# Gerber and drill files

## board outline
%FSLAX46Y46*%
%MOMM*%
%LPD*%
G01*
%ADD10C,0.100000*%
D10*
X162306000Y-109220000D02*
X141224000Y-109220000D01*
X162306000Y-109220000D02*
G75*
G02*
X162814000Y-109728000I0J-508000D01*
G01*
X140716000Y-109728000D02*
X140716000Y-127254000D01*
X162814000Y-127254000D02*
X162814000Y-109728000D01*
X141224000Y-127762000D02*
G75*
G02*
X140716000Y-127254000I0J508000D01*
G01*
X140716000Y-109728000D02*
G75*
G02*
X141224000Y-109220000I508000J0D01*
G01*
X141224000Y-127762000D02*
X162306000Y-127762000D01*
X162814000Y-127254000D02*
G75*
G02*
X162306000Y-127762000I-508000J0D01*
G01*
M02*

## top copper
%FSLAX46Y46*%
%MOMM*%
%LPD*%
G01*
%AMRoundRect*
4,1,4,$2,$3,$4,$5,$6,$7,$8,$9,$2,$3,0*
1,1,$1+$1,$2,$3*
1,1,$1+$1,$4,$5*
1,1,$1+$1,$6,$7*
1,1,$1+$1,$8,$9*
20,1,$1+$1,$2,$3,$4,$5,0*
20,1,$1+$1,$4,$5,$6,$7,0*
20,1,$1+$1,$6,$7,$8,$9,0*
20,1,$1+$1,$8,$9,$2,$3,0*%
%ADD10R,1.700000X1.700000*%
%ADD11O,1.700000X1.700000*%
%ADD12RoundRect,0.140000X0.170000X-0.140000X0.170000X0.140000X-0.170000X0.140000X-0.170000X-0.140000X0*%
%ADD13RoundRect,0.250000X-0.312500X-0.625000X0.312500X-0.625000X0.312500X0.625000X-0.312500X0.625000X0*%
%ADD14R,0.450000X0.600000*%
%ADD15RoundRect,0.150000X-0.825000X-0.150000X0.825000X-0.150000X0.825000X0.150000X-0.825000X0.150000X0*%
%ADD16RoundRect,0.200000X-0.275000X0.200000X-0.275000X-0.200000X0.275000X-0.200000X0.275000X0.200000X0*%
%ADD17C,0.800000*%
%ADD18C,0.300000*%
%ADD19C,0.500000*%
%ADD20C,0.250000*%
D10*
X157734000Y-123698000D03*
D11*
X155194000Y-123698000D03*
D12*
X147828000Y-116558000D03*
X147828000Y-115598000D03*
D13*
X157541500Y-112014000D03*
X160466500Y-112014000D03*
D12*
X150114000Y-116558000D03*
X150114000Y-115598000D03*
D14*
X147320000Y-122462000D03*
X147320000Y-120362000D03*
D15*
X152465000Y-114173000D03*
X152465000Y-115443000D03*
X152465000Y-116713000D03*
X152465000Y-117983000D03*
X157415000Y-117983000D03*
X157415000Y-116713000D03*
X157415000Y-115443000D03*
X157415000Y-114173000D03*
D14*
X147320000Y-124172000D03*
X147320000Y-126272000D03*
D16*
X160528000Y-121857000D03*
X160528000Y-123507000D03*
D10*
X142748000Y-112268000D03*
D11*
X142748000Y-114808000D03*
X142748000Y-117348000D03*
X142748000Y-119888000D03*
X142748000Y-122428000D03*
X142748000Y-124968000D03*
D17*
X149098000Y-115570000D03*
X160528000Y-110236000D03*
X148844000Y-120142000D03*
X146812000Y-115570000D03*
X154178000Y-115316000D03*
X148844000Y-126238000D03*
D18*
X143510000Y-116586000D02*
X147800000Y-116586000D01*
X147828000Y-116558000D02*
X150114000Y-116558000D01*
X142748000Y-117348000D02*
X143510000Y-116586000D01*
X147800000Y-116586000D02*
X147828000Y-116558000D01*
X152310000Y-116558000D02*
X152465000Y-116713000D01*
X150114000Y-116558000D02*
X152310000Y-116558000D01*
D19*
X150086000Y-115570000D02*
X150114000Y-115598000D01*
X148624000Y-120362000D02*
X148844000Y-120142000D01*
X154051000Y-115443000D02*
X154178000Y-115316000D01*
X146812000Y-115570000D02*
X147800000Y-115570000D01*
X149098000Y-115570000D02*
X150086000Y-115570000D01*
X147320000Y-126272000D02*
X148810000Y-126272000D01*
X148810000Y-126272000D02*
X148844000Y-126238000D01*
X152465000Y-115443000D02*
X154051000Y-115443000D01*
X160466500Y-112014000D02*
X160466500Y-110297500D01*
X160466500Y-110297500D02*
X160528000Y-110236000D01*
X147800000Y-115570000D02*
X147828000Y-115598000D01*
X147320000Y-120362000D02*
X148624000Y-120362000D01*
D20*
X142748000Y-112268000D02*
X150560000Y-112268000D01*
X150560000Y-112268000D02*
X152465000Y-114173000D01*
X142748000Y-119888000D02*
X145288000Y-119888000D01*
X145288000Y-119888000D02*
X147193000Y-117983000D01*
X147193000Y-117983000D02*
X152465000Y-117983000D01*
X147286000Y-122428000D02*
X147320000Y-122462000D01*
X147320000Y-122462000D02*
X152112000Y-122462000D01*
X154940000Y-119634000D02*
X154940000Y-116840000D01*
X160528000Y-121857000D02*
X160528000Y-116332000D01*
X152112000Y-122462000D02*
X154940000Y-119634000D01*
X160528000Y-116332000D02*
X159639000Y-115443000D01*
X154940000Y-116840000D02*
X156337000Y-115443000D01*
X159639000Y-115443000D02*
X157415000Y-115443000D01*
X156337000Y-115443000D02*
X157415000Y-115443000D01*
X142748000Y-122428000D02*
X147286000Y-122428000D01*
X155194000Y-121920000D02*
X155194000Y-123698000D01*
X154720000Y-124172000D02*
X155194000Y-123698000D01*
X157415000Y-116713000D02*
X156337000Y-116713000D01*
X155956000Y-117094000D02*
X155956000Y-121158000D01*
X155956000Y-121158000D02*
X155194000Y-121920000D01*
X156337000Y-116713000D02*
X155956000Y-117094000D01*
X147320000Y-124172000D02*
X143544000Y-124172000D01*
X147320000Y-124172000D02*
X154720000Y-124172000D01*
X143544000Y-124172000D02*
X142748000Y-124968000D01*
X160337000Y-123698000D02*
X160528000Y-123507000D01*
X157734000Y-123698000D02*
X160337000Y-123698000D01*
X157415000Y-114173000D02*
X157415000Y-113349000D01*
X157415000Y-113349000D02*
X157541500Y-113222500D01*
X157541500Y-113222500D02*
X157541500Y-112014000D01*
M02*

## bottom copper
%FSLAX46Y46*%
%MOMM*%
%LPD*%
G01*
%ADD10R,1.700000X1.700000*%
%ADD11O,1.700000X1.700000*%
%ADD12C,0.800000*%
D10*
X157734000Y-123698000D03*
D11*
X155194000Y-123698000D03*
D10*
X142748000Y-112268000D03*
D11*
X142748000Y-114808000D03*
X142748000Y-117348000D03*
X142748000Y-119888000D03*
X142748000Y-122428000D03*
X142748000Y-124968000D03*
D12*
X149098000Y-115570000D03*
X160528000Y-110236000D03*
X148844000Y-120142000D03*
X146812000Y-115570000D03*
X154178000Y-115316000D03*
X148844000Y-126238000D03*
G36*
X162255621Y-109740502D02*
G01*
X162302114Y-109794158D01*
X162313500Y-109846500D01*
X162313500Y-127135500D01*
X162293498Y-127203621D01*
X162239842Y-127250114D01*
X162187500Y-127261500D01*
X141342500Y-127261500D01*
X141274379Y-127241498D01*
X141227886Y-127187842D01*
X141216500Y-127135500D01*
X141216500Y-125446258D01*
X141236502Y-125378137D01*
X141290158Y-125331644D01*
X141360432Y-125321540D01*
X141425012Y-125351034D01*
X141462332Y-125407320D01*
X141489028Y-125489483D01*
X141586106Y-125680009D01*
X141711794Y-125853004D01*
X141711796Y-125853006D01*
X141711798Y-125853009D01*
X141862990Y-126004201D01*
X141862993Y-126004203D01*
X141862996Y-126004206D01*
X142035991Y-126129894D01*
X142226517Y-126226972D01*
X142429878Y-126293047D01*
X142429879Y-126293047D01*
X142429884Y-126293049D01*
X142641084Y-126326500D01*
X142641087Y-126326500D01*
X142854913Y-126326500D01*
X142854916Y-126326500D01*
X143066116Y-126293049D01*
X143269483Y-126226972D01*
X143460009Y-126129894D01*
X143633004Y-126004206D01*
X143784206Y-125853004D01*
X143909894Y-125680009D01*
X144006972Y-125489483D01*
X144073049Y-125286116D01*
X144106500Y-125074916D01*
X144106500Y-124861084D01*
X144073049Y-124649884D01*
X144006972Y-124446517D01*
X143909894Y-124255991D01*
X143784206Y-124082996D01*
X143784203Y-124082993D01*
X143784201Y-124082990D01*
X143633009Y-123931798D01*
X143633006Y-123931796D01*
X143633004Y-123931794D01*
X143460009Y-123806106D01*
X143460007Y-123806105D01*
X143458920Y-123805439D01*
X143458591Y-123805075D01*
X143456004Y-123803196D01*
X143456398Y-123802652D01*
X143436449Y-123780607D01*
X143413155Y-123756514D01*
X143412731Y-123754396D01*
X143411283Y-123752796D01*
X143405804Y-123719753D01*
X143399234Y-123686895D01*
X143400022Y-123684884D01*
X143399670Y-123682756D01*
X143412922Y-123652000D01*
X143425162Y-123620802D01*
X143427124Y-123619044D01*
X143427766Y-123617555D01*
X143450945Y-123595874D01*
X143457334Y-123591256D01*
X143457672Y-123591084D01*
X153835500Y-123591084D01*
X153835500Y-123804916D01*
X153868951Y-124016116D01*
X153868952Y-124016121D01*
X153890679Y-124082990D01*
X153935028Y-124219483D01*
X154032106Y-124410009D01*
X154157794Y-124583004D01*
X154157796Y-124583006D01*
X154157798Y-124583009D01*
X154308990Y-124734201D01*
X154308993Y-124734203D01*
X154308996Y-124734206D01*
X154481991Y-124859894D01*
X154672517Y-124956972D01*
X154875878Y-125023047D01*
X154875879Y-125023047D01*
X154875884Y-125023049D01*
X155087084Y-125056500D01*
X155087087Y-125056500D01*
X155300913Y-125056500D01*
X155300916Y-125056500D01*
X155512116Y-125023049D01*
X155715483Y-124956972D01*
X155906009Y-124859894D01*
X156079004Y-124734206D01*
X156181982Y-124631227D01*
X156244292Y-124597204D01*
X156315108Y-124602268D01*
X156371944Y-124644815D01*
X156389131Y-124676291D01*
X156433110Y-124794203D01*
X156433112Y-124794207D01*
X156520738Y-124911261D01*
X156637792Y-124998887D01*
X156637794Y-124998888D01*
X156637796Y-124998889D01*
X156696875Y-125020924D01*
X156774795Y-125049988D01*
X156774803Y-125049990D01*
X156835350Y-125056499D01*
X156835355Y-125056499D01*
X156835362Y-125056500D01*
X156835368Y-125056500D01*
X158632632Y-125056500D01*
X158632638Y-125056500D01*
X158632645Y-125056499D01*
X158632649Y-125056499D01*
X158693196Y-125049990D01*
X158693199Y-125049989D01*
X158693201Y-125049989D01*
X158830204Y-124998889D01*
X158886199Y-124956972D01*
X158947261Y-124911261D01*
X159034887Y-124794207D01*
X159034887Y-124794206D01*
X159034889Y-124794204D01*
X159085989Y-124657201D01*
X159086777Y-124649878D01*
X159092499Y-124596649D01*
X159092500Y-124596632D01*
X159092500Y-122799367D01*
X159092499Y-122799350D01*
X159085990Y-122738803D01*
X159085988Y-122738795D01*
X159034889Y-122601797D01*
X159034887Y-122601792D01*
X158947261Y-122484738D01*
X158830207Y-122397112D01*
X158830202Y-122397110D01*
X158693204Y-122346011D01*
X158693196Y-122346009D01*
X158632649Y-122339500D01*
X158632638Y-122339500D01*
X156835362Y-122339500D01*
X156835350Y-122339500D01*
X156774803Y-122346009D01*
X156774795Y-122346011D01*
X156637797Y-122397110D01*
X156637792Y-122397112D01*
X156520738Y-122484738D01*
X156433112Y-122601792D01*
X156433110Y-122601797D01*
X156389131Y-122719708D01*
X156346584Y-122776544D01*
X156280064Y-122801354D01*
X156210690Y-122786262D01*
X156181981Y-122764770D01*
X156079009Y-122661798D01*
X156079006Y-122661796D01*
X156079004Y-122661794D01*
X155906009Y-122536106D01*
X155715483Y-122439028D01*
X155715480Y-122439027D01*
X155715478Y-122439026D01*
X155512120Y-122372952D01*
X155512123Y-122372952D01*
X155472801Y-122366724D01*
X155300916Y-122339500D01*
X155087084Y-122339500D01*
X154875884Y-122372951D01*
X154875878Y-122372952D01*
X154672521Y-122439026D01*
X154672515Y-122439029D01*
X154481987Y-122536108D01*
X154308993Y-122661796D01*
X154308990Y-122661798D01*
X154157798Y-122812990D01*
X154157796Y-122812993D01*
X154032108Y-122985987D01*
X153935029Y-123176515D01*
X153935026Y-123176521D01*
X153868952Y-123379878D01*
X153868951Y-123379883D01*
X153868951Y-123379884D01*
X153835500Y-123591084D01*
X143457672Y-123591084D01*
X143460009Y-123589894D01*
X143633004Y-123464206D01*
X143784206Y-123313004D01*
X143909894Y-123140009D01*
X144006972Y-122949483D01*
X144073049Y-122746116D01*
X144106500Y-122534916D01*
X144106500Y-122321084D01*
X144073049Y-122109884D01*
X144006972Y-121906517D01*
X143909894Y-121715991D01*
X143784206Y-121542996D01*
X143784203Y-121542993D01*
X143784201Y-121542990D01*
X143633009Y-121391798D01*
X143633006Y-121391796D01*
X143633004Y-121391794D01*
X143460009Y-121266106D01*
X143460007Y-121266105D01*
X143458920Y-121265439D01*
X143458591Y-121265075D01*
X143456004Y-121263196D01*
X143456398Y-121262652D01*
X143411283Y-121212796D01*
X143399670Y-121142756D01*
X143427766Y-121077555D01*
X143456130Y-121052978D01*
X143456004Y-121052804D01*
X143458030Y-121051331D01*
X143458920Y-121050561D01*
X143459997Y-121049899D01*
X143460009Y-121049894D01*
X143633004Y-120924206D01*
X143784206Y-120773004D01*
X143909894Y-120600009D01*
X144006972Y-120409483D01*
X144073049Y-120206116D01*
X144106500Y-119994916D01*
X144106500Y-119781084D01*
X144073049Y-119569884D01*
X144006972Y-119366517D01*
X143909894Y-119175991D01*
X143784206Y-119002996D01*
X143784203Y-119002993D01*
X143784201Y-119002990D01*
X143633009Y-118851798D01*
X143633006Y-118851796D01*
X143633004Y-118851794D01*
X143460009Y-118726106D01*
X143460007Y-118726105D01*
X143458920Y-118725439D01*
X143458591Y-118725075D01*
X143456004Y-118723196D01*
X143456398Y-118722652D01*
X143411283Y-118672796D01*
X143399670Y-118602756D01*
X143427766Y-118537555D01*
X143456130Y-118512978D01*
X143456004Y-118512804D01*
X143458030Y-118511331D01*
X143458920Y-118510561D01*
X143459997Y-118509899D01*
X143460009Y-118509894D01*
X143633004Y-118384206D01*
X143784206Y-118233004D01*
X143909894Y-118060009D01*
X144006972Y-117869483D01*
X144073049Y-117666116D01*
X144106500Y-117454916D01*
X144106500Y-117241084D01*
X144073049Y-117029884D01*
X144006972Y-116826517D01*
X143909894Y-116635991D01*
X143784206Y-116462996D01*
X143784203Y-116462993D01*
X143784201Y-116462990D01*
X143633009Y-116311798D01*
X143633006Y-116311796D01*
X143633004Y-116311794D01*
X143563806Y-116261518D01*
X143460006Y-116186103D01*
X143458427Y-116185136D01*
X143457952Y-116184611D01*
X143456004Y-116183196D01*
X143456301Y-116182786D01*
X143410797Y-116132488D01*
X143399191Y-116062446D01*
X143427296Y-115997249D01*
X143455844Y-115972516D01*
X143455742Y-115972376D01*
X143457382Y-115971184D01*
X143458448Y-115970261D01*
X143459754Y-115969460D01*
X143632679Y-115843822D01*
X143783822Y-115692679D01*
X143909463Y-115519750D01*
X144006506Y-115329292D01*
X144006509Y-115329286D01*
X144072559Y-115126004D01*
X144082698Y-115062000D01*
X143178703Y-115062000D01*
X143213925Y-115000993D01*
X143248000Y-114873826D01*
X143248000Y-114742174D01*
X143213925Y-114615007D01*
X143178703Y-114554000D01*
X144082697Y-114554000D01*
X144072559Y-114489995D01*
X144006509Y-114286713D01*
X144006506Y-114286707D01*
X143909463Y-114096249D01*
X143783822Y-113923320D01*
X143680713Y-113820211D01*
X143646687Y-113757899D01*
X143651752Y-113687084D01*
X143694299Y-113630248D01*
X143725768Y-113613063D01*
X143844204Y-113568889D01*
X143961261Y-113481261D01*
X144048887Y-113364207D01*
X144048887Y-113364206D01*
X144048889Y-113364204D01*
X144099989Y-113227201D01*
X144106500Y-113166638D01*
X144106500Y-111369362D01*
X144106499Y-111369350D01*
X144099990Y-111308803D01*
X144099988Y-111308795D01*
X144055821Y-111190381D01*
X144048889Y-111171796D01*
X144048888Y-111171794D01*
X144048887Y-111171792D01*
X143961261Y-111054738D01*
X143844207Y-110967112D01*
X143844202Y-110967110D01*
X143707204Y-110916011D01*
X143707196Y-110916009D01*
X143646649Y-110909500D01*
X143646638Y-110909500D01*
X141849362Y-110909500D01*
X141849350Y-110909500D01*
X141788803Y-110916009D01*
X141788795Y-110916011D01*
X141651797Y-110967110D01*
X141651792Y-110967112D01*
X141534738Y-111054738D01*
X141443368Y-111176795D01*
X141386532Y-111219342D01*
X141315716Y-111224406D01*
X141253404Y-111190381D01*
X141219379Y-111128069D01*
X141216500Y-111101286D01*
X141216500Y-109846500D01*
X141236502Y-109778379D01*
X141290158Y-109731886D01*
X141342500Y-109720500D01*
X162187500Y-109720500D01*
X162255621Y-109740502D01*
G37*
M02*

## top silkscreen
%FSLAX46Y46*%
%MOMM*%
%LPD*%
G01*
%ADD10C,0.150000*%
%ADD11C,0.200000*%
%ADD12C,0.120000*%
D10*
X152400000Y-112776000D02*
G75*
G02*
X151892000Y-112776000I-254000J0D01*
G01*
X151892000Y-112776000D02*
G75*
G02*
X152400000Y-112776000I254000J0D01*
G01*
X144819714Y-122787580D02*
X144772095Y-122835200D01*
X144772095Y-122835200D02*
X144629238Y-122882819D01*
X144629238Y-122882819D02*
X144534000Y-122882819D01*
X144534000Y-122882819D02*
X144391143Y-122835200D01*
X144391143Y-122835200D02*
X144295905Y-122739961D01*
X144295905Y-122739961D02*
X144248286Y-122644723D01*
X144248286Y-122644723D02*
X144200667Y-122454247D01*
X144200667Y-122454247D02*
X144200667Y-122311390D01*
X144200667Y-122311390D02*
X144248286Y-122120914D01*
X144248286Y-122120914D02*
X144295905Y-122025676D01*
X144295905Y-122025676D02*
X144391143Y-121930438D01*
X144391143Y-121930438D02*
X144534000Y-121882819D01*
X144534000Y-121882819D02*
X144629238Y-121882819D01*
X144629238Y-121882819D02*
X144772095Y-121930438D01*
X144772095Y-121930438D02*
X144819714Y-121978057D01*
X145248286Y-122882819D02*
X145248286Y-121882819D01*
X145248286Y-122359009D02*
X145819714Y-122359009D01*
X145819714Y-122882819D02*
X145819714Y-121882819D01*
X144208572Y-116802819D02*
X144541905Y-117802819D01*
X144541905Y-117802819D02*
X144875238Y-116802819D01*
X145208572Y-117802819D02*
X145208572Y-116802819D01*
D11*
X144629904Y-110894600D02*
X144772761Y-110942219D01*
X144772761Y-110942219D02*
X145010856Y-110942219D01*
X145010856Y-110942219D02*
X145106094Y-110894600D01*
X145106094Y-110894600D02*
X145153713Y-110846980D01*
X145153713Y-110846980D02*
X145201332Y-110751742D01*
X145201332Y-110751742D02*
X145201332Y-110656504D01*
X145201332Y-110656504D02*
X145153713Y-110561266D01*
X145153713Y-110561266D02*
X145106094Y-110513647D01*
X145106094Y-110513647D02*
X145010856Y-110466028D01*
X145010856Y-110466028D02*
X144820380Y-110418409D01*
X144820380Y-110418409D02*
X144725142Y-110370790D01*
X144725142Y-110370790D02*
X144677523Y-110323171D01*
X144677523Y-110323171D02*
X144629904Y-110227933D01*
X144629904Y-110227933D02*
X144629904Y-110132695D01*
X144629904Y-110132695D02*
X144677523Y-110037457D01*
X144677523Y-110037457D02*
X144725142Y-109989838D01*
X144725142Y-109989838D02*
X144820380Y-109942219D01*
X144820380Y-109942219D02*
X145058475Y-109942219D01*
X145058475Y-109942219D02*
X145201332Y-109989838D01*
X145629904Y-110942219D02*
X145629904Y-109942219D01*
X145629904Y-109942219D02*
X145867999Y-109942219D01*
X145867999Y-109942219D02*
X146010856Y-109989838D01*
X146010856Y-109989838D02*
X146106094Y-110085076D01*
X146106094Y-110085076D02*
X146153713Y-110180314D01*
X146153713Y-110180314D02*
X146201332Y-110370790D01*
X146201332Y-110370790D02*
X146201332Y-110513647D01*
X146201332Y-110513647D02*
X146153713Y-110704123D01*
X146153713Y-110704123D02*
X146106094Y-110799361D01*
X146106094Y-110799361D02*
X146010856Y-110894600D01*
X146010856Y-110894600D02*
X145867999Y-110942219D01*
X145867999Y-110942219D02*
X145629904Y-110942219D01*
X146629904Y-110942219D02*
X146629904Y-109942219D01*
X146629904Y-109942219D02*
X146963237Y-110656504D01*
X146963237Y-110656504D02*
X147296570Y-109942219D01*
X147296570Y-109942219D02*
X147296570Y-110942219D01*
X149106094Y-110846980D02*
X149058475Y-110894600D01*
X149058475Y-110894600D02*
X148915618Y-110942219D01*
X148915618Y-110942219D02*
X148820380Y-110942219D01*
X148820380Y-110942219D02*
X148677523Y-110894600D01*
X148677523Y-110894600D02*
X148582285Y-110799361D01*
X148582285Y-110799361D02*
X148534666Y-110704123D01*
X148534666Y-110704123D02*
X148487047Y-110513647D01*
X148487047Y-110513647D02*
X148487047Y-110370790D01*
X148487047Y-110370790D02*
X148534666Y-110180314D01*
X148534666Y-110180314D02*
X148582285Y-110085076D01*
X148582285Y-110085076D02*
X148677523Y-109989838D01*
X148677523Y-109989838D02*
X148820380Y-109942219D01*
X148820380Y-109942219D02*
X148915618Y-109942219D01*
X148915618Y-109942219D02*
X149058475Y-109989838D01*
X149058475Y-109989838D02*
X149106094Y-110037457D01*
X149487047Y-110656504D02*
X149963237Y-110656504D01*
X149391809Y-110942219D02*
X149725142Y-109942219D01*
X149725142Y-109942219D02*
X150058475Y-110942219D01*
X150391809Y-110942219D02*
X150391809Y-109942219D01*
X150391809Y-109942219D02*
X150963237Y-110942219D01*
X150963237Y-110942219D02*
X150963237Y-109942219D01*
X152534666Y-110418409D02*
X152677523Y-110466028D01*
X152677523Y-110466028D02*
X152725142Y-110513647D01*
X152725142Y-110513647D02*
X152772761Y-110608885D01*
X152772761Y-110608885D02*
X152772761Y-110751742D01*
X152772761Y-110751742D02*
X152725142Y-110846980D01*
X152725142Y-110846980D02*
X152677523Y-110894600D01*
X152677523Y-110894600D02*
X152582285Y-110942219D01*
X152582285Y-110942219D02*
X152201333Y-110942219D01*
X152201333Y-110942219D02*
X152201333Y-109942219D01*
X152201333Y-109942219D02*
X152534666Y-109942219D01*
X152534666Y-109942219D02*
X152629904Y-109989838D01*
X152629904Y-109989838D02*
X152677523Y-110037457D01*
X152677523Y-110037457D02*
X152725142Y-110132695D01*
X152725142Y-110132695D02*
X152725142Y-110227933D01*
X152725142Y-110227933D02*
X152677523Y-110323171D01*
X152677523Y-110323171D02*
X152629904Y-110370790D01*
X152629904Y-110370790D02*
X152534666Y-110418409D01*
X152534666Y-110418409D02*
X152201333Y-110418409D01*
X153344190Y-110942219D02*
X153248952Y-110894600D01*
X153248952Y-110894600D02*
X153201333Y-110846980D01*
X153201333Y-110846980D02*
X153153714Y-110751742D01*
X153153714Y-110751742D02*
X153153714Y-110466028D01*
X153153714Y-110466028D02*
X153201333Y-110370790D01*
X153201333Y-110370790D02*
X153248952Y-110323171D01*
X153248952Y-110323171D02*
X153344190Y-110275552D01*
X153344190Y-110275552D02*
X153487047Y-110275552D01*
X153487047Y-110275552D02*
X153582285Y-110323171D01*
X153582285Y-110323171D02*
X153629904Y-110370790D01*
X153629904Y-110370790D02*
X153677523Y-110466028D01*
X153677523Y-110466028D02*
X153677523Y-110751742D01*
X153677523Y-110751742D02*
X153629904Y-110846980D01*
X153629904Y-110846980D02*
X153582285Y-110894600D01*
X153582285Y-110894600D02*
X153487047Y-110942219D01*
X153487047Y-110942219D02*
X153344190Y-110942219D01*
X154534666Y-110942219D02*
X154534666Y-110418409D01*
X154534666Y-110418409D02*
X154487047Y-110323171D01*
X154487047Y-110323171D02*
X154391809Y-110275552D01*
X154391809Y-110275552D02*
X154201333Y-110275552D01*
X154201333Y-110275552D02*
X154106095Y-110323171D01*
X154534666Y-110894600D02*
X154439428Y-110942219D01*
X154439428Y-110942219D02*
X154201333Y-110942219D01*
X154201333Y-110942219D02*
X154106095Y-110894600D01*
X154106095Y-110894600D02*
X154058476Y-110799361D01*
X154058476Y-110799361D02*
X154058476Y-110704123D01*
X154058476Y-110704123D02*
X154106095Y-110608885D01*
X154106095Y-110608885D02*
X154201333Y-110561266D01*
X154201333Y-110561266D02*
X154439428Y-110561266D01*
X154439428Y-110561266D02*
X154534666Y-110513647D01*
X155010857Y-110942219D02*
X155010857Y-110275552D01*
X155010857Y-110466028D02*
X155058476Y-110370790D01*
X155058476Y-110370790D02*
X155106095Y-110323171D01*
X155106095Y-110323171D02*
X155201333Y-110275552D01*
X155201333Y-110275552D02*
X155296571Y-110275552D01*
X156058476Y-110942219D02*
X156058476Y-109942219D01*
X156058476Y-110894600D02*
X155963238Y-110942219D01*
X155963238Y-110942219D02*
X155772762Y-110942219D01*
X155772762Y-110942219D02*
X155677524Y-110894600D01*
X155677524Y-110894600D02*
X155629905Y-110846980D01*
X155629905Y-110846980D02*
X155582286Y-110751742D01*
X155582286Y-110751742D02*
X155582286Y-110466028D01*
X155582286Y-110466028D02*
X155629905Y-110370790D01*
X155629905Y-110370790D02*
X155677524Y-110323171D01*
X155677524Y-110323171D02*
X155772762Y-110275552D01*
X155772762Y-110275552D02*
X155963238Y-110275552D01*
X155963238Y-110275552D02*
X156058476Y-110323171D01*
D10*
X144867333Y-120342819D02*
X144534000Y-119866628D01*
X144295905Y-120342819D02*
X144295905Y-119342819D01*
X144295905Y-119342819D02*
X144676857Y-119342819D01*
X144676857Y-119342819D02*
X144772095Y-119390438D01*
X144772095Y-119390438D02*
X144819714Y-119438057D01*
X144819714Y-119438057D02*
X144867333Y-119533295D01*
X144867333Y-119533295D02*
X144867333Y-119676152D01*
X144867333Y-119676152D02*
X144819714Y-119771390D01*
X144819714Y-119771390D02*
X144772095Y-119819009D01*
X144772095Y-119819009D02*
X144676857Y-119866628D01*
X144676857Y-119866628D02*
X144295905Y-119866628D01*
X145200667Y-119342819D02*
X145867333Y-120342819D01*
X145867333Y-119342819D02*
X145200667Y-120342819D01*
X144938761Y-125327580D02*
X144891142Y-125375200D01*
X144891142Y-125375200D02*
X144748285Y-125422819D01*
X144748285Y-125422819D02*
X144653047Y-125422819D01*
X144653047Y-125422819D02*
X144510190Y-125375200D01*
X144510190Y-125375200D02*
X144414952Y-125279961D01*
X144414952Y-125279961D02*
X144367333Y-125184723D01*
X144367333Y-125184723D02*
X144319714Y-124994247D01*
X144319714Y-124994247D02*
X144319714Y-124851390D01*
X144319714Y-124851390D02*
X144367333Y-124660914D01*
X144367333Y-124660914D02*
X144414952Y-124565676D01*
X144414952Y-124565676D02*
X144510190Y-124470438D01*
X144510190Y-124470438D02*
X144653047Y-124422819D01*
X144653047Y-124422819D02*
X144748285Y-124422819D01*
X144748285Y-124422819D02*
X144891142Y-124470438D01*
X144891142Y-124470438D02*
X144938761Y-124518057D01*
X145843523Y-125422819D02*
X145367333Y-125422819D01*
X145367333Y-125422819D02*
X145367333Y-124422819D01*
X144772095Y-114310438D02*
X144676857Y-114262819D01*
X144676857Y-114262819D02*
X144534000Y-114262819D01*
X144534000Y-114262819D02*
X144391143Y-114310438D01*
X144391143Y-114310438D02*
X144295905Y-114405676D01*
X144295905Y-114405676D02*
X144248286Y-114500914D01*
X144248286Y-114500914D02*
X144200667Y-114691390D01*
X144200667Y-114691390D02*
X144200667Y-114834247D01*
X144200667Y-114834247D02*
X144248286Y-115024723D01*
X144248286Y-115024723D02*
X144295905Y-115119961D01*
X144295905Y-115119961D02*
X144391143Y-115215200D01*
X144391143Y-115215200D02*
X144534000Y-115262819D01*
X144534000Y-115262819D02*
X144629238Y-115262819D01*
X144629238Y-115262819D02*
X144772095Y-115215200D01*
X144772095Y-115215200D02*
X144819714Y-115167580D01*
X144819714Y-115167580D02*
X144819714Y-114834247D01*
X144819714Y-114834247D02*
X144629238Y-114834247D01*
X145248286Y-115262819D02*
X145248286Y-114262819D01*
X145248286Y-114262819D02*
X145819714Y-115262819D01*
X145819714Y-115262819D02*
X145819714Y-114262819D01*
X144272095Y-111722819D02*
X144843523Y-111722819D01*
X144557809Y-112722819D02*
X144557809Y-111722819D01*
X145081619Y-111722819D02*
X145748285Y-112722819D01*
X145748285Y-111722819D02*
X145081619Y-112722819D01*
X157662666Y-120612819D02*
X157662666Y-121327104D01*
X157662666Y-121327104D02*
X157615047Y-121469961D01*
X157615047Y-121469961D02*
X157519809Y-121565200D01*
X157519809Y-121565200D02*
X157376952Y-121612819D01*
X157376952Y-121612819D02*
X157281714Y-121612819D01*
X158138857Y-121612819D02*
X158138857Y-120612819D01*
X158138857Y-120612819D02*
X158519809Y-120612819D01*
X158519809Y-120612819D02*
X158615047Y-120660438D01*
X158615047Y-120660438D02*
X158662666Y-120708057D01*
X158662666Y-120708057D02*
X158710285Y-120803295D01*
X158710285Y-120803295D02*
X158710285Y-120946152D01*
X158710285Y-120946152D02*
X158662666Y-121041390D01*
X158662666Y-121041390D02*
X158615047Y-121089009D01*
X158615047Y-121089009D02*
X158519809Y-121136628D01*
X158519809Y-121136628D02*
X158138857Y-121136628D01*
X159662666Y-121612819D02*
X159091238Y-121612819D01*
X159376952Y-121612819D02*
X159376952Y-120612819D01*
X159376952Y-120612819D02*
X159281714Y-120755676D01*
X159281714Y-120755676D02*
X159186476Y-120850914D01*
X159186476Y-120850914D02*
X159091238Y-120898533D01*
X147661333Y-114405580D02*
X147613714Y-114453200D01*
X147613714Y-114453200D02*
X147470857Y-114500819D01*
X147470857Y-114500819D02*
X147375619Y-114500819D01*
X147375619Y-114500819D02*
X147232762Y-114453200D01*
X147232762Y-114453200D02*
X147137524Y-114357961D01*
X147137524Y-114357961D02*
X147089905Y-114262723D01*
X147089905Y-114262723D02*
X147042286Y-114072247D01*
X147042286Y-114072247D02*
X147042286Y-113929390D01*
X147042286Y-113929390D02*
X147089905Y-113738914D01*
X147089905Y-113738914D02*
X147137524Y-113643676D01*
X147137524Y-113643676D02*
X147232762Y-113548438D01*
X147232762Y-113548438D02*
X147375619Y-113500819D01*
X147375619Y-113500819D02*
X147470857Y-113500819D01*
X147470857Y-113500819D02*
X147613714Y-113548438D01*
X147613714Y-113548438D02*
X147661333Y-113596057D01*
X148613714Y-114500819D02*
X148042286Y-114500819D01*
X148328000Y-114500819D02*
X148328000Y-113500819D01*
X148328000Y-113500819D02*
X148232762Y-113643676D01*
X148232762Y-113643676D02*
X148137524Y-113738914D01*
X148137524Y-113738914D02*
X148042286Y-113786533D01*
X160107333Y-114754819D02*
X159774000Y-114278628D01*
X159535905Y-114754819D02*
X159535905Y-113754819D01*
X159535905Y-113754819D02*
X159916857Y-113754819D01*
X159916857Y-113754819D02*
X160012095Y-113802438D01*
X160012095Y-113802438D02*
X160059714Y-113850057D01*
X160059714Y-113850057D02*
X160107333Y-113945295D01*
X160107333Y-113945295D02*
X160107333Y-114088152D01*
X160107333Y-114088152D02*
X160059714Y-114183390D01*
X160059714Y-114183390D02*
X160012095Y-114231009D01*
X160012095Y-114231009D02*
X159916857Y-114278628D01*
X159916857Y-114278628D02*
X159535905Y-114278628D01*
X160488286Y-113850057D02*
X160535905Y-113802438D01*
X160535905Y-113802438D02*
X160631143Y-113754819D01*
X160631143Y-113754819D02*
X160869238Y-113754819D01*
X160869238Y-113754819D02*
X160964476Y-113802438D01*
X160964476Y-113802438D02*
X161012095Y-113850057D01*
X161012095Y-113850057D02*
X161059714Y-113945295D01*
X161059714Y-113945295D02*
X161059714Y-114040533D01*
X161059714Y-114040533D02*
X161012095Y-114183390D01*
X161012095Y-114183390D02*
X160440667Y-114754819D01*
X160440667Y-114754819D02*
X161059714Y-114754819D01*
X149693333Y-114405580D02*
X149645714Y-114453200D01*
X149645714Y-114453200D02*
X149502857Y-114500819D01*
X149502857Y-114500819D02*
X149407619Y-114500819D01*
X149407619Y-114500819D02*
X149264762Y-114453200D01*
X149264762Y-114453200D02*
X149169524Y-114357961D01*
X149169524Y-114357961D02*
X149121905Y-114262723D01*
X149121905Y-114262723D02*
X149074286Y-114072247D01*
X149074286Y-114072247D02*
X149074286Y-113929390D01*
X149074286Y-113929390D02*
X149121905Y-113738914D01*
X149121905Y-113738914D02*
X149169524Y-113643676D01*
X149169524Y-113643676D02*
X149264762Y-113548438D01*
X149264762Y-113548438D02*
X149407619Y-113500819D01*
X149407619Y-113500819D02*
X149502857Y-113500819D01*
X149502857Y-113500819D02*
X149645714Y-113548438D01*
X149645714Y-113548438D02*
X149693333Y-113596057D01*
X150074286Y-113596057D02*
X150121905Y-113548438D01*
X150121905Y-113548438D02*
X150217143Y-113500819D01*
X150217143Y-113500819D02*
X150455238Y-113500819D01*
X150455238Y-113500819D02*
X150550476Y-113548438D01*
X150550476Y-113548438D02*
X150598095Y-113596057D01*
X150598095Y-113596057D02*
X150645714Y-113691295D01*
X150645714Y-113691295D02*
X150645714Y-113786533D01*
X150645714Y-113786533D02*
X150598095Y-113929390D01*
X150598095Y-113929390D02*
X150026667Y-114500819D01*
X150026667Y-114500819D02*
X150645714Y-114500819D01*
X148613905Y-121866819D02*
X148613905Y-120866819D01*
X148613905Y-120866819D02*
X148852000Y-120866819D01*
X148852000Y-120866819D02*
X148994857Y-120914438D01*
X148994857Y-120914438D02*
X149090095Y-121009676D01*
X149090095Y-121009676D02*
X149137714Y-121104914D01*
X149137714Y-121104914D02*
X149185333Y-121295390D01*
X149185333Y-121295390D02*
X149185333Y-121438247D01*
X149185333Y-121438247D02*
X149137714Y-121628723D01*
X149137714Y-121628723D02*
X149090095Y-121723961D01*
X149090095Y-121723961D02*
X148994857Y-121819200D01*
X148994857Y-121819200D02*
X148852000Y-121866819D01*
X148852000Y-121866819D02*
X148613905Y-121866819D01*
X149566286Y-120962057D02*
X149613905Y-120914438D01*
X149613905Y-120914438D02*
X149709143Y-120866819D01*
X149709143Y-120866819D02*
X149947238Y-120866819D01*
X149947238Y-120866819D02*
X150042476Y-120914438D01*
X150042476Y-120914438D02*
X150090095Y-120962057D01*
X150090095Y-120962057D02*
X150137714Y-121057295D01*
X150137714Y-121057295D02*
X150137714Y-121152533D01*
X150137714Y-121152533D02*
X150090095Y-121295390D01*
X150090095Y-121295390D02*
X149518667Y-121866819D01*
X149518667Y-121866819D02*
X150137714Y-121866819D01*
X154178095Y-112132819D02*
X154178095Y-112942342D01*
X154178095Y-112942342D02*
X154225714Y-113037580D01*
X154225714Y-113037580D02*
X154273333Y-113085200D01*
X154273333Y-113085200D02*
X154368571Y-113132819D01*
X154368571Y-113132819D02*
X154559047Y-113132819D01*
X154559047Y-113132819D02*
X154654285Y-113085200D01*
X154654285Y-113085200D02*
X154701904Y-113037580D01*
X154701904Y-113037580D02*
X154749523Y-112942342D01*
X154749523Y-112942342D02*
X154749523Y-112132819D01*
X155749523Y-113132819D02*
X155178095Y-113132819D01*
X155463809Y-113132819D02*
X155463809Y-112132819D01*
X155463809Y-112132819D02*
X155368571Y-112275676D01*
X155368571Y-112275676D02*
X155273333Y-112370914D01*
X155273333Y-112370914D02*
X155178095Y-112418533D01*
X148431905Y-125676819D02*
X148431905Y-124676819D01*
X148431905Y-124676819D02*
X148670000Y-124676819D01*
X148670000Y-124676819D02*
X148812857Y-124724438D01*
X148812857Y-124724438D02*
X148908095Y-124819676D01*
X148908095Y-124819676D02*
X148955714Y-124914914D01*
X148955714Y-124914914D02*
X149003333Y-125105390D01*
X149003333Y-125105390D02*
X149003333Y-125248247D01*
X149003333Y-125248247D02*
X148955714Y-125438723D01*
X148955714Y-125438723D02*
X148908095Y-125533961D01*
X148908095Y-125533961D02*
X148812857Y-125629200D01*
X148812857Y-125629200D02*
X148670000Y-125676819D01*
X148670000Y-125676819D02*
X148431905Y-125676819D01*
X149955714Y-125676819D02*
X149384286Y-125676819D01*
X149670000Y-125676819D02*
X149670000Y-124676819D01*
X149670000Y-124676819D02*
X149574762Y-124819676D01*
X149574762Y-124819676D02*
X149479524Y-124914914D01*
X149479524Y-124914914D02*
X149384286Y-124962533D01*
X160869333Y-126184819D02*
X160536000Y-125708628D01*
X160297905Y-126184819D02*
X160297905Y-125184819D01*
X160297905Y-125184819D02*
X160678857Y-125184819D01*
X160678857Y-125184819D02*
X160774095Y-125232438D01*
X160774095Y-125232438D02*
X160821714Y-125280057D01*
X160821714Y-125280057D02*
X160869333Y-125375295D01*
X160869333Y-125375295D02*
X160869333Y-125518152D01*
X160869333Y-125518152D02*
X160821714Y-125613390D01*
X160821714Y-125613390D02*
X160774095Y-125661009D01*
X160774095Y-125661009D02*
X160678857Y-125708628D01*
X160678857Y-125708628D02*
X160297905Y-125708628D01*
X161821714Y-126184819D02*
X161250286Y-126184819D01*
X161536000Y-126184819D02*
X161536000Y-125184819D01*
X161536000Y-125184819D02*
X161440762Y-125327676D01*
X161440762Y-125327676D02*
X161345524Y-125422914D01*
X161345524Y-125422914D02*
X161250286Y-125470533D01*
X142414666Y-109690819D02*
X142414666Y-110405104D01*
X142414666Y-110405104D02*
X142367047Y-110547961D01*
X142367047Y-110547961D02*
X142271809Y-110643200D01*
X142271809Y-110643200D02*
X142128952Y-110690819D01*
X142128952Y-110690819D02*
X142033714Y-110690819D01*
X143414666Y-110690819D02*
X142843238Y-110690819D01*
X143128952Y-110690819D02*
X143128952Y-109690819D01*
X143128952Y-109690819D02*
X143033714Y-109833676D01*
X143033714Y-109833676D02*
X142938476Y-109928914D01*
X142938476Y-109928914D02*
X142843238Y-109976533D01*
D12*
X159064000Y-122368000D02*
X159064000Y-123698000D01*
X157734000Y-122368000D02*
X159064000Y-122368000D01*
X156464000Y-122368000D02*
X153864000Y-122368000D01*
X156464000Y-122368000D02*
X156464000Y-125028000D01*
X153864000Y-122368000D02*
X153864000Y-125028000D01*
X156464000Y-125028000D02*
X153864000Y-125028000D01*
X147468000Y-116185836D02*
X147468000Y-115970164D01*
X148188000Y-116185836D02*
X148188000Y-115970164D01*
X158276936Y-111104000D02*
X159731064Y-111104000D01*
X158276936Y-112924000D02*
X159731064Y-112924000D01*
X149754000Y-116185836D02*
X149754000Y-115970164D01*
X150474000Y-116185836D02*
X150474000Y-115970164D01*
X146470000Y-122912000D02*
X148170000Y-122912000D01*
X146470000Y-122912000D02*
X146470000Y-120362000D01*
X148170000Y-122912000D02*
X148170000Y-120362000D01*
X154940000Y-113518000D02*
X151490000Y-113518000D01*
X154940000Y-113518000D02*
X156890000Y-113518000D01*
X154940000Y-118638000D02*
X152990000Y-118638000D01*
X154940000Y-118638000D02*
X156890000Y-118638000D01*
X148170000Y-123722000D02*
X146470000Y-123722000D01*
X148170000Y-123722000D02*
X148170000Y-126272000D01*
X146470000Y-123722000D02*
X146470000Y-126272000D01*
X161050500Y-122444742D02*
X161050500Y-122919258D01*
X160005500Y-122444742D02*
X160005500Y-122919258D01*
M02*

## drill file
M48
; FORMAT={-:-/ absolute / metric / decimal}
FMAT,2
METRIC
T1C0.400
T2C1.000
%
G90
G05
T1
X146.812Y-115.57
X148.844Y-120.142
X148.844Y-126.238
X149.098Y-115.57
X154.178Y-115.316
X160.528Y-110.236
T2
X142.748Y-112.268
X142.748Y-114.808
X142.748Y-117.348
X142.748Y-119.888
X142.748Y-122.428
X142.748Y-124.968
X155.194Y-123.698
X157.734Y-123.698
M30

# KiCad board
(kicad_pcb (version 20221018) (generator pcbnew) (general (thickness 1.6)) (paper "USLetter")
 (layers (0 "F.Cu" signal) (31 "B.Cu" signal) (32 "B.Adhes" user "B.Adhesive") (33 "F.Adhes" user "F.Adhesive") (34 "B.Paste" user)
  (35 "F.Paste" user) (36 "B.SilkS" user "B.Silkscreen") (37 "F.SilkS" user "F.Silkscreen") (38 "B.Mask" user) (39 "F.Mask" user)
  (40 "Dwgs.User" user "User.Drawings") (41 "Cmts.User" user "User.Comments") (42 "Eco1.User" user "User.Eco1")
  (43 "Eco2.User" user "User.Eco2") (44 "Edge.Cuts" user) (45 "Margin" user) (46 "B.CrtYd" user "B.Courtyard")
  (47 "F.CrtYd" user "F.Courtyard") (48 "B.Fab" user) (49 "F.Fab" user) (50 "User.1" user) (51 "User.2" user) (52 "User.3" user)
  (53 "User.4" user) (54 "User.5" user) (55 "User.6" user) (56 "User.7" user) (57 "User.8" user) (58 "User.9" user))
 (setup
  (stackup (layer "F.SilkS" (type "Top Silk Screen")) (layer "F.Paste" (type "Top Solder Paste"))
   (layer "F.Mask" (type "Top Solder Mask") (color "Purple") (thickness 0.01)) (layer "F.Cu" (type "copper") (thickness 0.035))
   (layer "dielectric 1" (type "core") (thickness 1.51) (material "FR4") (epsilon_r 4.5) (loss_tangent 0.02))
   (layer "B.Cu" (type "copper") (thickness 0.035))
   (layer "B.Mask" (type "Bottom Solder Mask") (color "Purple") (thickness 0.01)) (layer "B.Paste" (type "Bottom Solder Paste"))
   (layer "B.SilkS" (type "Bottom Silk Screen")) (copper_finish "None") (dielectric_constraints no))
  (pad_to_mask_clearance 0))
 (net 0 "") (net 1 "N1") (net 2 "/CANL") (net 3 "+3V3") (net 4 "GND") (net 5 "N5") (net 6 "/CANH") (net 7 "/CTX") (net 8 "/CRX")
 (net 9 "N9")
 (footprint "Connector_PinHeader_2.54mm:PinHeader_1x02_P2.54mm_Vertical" (layer "F.Cu") (at 157.734 123.698 -90)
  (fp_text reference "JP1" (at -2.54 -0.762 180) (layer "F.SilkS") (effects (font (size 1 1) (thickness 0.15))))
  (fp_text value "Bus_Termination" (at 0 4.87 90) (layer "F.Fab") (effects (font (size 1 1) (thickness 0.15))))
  (fp_line (start -1.33 -1.33) (end 0 -1.33) (stroke (width 0.12) (type solid)) (layer "F.SilkS"))
  (fp_line (start -1.33 0) (end -1.33 -1.33) (stroke (width 0.12) (type solid)) (layer "F.SilkS"))
  (fp_line (start -1.33 1.27) (end -1.33 3.87) (stroke (width 0.12) (type solid)) (layer "F.SilkS"))
  (fp_line (start -1.33 1.27) (end 1.33 1.27) (stroke (width 0.12) (type solid)) (layer "F.SilkS"))
  (fp_line (start -1.33 3.87) (end 1.33 3.87) (stroke (width 0.12) (type solid)) (layer "F.SilkS"))
  (fp_line (start 1.33 1.27) (end 1.33 3.87) (stroke (width 0.12) (type solid)) (layer "F.SilkS"))
  (pad "1" thru_hole rect (at 0 0 270) (size 1.7 1.7) (drill 1) (layers "*.Cu" "*.Mask") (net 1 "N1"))
  (pad "2" thru_hole oval (at 0 2.54 270) (size 1.7 1.7) (drill 1) (layers "*.Cu" "*.Mask") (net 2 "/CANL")))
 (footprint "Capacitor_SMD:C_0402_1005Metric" (layer "F.Cu") (at 147.828 116.078 90)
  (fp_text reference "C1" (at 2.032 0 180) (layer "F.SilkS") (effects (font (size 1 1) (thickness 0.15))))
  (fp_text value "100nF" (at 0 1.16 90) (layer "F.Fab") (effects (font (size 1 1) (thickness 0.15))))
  (fp_line (start -0.107836 -0.36) (end 0.107836 -0.36) (stroke (width 0.12) (type solid)) (layer "F.SilkS"))
  (fp_line (start -0.107836 0.36) (end 0.107836 0.36) (stroke (width 0.12) (type solid)) (layer "F.SilkS"))
  (pad "1" smd roundrect (at -0.48 0 90) (size 0.56 0.62) (layers "F.Cu" "F.Paste" "F.Mask") (roundrect_rratio 0.25) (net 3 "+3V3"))
  (pad "2" smd roundrect (at 0.48 0 90) (size 0.56 0.62) (layers "F.Cu" "F.Paste" "F.Mask") (roundrect_rratio 0.25) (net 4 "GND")))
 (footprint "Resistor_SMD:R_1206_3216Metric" (layer "F.Cu") (at 159.004 112.014)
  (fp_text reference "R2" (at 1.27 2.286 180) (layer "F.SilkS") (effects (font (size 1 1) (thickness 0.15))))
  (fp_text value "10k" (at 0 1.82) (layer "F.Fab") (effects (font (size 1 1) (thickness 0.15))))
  (fp_line (start -0.727064 -0.91) (end 0.727064 -0.91) (stroke (width 0.12) (type solid)) (layer "F.SilkS"))
  (fp_line (start -0.727064 0.91) (end 0.727064 0.91) (stroke (width 0.12) (type solid)) (layer "F.SilkS"))
  (pad "1" smd roundrect (at -1.4625 0) (size 1.125 1.75) (layers "F.Cu" "F.Paste" "F.Mask") (roundrect_rratio 0.2222222222) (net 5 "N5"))
  (pad "2" smd roundrect (at 1.4625 0) (size 1.125 1.75) (layers "F.Cu" "F.Paste" "F.Mask") (roundrect_rratio 0.2222222222) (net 4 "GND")))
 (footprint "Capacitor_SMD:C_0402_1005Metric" (layer "F.Cu") (at 150.114 116.078 90)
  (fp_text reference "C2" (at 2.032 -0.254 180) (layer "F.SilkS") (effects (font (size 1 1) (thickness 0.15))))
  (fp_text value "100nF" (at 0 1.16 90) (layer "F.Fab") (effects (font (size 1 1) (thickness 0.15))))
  (fp_line (start -0.107836 -0.36) (end 0.107836 -0.36) (stroke (width 0.12) (type solid)) (layer "F.SilkS"))
  (fp_line (start -0.107836 0.36) (end 0.107836 0.36) (stroke (width 0.12) (type solid)) (layer "F.SilkS"))
  (pad "1" smd roundrect (at -0.48 0 90) (size 0.56 0.62) (layers "F.Cu" "F.Paste" "F.Mask") (roundrect_rratio 0.25) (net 3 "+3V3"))
  (pad "2" smd roundrect (at 0.48 0 90) (size 0.56 0.62) (layers "F.Cu" "F.Paste" "F.Mask") (roundrect_rratio 0.25) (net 4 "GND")))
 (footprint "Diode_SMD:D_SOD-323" (layer "F.Cu") (at 147.32 121.412 90)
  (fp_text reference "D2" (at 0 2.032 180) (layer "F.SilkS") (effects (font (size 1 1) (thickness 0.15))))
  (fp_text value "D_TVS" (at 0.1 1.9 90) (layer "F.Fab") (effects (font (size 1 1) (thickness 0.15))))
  (fp_line (start -1.5 -0.85) (end -1.5 0.85) (stroke (width 0.12) (type solid)) (layer "F.SilkS"))
  (fp_line (start -1.5 -0.85) (end 1.05 -0.85) (stroke (width 0.12) (type solid)) (layer "F.SilkS"))
  (fp_line (start -1.5 0.85) (end 1.05 0.85) (stroke (width 0.12) (type solid)) (layer "F.SilkS"))
  (pad "1" smd rect (at -1.05 0 90) (size 0.6 0.45) (layers "F.Cu" "F.Paste" "F.Mask") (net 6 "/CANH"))
  (pad "2" smd rect (at 1.05 0 90) (size 0.6 0.45) (layers "F.Cu" "F.Paste" "F.Mask") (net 4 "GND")))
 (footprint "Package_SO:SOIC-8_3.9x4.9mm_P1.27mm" (layer "F.Cu") (at 154.94 116.078)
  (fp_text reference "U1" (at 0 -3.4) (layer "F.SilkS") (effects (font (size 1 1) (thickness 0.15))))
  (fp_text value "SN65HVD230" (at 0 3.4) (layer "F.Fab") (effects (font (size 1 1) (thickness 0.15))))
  (fp_line (start 0 -2.56) (end -3.45 -2.56) (stroke (width 0.12) (type solid)) (layer "F.SilkS"))
  (fp_line (start 0 -2.56) (end 1.95 -2.56) (stroke (width 0.12) (type solid)) (layer "F.SilkS"))
  (fp_line (start 0 2.56) (end -1.95 2.56) (stroke (width 0.12) (type solid)) (layer "F.SilkS"))
  (fp_line (start 0 2.56) (end 1.95 2.56) (stroke (width 0.12) (type solid)) (layer "F.SilkS"))
  (pad "1" smd roundrect (at -2.475 -1.905) (size 1.95 0.6) (layers "F.Cu" "F.Paste" "F.Mask") (roundrect_rratio 0.25) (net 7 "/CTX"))
  (pad "2" smd roundrect (at -2.475 -0.635) (size 1.95 0.6) (layers "F.Cu" "F.Paste" "F.Mask") (roundrect_rratio 0.25) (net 4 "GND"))
  (pad "3" smd roundrect (at -2.475 0.635) (size 1.95 0.6) (layers "F.Cu" "F.Paste" "F.Mask") (roundrect_rratio 0.25) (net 3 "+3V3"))
  (pad "4" smd roundrect (at -2.475 1.905) (size 1.95 0.6) (layers "F.Cu" "F.Paste" "F.Mask") (roundrect_rratio 0.25) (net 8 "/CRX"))
  (pad "5" smd roundrect (at 2.475 1.905) (size 1.95 0.6) (layers "F.Cu" "F.Paste" "F.Mask") (roundrect_rratio 0.25) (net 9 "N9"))
  (pad "6" smd roundrect (at 2.475 0.635) (size 1.95 0.6) (layers "F.Cu" "F.Paste" "F.Mask") (roundrect_rratio 0.25) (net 2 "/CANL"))
  (pad "7" smd roundrect (at 2.475 -0.635) (size 1.95 0.6) (layers "F.Cu" "F.Paste" "F.Mask") (roundrect_rratio 0.25) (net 6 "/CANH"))
  (pad "8" smd roundrect (at 2.475 -1.905) (size 1.95 0.6) (layers "F.Cu" "F.Paste" "F.Mask") (roundrect_rratio 0.25) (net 5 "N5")))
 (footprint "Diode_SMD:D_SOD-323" (layer "F.Cu") (at 147.32 125.222 -90)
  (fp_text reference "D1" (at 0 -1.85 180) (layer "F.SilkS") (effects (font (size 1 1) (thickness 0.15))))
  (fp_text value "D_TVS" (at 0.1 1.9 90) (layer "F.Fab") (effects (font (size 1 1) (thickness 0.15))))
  (fp_line (start -1.5 -0.85) (end -1.5 0.85) (stroke (width 0.12) (type solid)) (layer "F.SilkS"))
  (fp_line (start -1.5 -0.85) (end 1.05 -0.85) (stroke (width 0.12) (type solid)) (layer "F.SilkS"))
  (fp_line (start -1.5 0.85) (end 1.05 0.85) (stroke (width 0.12) (type solid)) (layer "F.SilkS"))
  (pad "1" smd rect (at -1.05 0 270) (size 0.6 0.45) (layers "F.Cu" "F.Paste" "F.Mask") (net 2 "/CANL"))
  (pad "2" smd rect (at 1.05 0 270) (size 0.6 0.45) (layers "F.Cu" "F.Paste" "F.Mask") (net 4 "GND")))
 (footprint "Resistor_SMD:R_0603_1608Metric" (layer "F.Cu") (at 160.528 122.682 -90)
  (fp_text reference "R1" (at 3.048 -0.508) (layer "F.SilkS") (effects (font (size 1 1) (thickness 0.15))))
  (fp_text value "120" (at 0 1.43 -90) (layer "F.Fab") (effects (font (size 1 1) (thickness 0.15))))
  (fp_line (start -0.237258 -0.5225) (end 0.237258 -0.5225) (stroke (width 0.12) (type solid)) (layer "F.SilkS"))
  (fp_line (start -0.237258 0.5225) (end 0.237258 0.5225) (stroke (width 0.12) (type solid)) (layer "F.SilkS"))
  (pad "1" smd roundrect (at -0.825 0 270) (size 0.8 0.95) (layers "F.Cu" "F.Paste" "F.Mask") (roundrect_rratio 0.25) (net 6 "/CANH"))
  (pad "2" smd roundrect (at 0.825 0 270) (size 0.8 0.95) (layers "F.Cu" "F.Paste" "F.Mask") (roundrect_rratio 0.25) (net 1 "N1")))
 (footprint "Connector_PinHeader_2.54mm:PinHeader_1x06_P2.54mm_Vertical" (layer "B.Cu") (at 142.748 112.268 180)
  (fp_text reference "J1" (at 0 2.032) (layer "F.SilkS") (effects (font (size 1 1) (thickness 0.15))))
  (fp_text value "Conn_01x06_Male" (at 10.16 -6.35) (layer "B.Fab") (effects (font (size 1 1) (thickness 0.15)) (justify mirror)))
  (pad "1" thru_hole rect (at 0 0 180) (size 1.7 1.7) (drill 1) (layers "*.Cu" "*.Mask") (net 7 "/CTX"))
  (pad "2" thru_hole oval (at 0 -2.54 180) (size 1.7 1.7) (drill 1) (layers "*.Cu" "*.Mask") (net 4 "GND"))
  (pad "3" thru_hole oval (at 0 -5.08 180) (size 1.7 1.7) (drill 1) (layers "*.Cu" "*.Mask") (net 3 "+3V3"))
  (pad "4" thru_hole oval (at 0 -7.62 180) (size 1.7 1.7) (drill 1) (layers "*.Cu" "*.Mask") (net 8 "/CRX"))
  (pad "5" thru_hole oval (at 0 -10.16 180) (size 1.7 1.7) (drill 1) (layers "*.Cu" "*.Mask") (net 6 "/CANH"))
  (pad "6" thru_hole oval (at 0 -12.7 180) (size 1.7 1.7) (drill 1) (layers "*.Cu" "*.Mask") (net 2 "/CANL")))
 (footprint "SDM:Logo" (layer "B.Cu") (at 156.718 118.364 180)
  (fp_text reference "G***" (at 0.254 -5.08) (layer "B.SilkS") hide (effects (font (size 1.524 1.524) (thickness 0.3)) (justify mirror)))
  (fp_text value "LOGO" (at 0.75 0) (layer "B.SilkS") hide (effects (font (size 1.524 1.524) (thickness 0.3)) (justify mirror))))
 (gr_circle (center 152.146 112.776) (end 152.146 112.522) (stroke (width 0.15) (type solid)) (fill none) (layer "F.SilkS"))
 (gr_line (start 162.306 109.22) (end 141.224 109.22) (stroke (width 0.1) (type solid)) (layer "Edge.Cuts"))
 (gr_arc (start 162.306 109.22) (mid 162.66521 109.36879) (end 162.814 109.728) (stroke (width 0.1) (type solid)) (layer "Edge.Cuts"))
 (gr_line (start 140.716 109.728) (end 140.716 127.254) (stroke (width 0.1) (type solid)) (layer "Edge.Cuts"))
 (gr_line (start 162.814 127.254) (end 162.814 109.728) (stroke (width 0.1) (type solid)) (layer "Edge.Cuts"))
 (gr_arc (start 141.224 127.762) (mid 140.86479 127.61321) (end 140.716 127.254) (stroke (width 0.1) (type solid)) (layer "Edge.Cuts"))
 (gr_arc (start 140.716 109.728) (mid 140.86479 109.36879) (end 141.224 109.22) (stroke (width 0.1) (type solid)) (layer "Edge.Cuts"))
 (gr_line (start 141.224 127.762) (end 162.306 127.762) (stroke (width 0.1) (type solid)) (layer "Edge.Cuts"))
 (gr_arc (start 162.814 127.254) (mid 162.66521 127.61321) (end 162.306 127.762) (stroke (width 0.1) (type solid)) (layer "Edge.Cuts"))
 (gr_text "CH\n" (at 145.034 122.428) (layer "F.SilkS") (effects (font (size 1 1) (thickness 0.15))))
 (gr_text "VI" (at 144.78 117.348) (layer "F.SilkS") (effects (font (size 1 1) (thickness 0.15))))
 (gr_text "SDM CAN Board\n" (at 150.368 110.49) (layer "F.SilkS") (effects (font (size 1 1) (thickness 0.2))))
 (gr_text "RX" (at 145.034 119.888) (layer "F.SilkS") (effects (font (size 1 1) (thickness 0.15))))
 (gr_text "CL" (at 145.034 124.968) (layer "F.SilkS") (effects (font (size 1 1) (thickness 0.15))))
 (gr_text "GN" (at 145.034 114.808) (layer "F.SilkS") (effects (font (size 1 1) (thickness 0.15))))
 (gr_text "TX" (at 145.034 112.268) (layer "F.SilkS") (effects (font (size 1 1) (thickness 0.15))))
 (segment (start 143.51 116.586) (end 147.8 116.586) (width 0.3) (layer "F.Cu") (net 3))
 (segment (start 147.828 116.558) (end 150.114 116.558) (width 0.3) (layer "F.Cu") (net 3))
 (segment (start 142.748 117.348) (end 143.51 116.586) (width 0.3) (layer "F.Cu") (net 3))
 (segment (start 147.8 116.586) (end 147.828 116.558) (width 0.3) (layer "F.Cu") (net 3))
 (segment (start 152.31 116.558) (end 152.465 116.713) (width 0.3) (layer "F.Cu") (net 3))
 (segment (start 150.114 116.558) (end 152.31 116.558) (width 0.3) (layer "F.Cu") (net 3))
 (segment (start 150.086 115.57) (end 150.114 115.598) (width 0.5) (layer "F.Cu") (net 4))
 (segment (start 148.624 120.362) (end 148.844 120.142) (width 0.5) (layer "F.Cu") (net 4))
 (segment (start 154.051 115.443) (end 154.178 115.316) (width 0.5) (layer "F.Cu") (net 4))
 (segment (start 146.812 115.57) (end 147.8 115.57) (width 0.5) (layer "F.Cu") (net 4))
 (segment (start 149.098 115.57) (end 150.086 115.57) (width 0.5) (layer "F.Cu") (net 4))
 (segment (start 147.32 126.272) (end 148.81 126.272) (width 0.5) (layer "F.Cu") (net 4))
 (segment (start 148.81 126.272) (end 148.844 126.238) (width 0.5) (layer "F.Cu") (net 4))
 (segment (start 152.465 115.443) (end 154.051 115.443) (width 0.5) (layer "F.Cu") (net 4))
 (segment (start 160.4665 112.014) (end 160.4665 110.2975) (width 0.5) (layer "F.Cu") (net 4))
 (segment (start 160.4665 110.2975) (end 160.528 110.236) (width 0.5) (layer "F.Cu") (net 4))
 (segment (start 147.8 115.57) (end 147.828 115.598) (width 0.5) (layer "F.Cu") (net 4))
 (segment (start 147.32 120.362) (end 148.624 120.362) (width 0.5) (layer "F.Cu") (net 4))
 (via (at 149.098 115.57) (size 0.8) (drill 0.4) (layers "F.Cu" "B.Cu") (free) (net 4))
 (via (at 160.528 110.236) (size 0.8) (drill 0.4) (layers "F.Cu" "B.Cu") (free) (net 4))
 (via (at 148.844 120.142) (size 0.8) (drill 0.4) (layers "F.Cu" "B.Cu") (free) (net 4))
 (via (at 146.812 115.57) (size 0.8) (drill 0.4) (layers "F.Cu" "B.Cu") (free) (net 4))
 (via (at 154.178 115.316) (size 0.8) (drill 0.4) (layers "F.Cu" "B.Cu") (free) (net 4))
 (via (at 148.844 126.238) (size 0.8) (drill 0.4) (layers "F.Cu" "B.Cu") (free) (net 4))
 (segment (start 142.748 112.268) (end 150.56 112.268) (width 0.25) (layer "F.Cu") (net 7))
 (segment (start 150.56 112.268) (end 152.465 114.173) (width 0.25) (layer "F.Cu") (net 7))
 (segment (start 142.748 119.888) (end 145.288 119.888) (width 0.25) (layer "F.Cu") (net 8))
 (segment (start 145.288 119.888) (end 147.193 117.983) (width 0.25) (layer "F.Cu") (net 8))
 (segment (start 147.193 117.983) (end 152.465 117.983) (width 0.25) (layer "F.Cu") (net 8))
 (segment (start 147.286 122.428) (end 147.32 122.462) (width 0.25) (layer "F.Cu") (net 6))
 (segment (start 147.32 122.462) (end 152.112 122.462) (width 0.25) (layer "F.Cu") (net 6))
 (segment (start 154.94 119.634) (end 154.94 116.84) (width 0.25) (layer "F.Cu") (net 6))
 (segment (start 160.528 121.857) (end 160.528 116.332) (width 0.25) (layer "F.Cu") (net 6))
 (segment (start 152.112 122.462) (end 154.94 119.634) (width 0.25) (layer "F.Cu") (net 6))
 (segment (start 160.528 116.332) (end 159.639 115.443) (width 0.25) (layer "F.Cu") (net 6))
 (segment (start 154.94 116.84) (end 156.337 115.443) (width 0.25) (layer "F.Cu") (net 6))
 (segment (start 159.639 115.443) (end 157.415 115.443) (width 0.25) (layer "F.Cu") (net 6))
 (segment (start 156.337 115.443) (end 157.415 115.443) (width 0.25) (layer "F.Cu") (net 6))
 (segment (start 142.748 122.428) (end 147.286 122.428) (width 0.25) (layer "F.Cu") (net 6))
 (segment (start 155.194 121.92) (end 155.194 123.698) (width 0.25) (layer "F.Cu") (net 2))
 (segment (start 154.72 124.172) (end 155.194 123.698) (width 0.25) (layer "F.Cu") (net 2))
 (segment (start 157.415 116.713) (end 156.337 116.713) (width 0.25) (layer "F.Cu") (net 2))
 (segment (start 155.956 117.094) (end 155.956 121.158) (width 0.25) (layer "F.Cu") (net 2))
 (segment (start 155.956 121.158) (end 155.194 121.92) (width 0.25) (layer "F.Cu") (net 2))
 (segment (start 156.337 116.713) (end 155.956 117.094) (width 0.25) (layer "F.Cu") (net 2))
 (segment (start 147.32 124.172) (end 143.544 124.172) (width 0.25) (layer "F.Cu") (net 2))
 (segment (start 147.32 124.172) (end 154.72 124.172) (width 0.25) (layer "F.Cu") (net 2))
 (segment (start 143.544 124.172) (end 142.748 124.968) (width 0.25) (layer "F.Cu") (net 2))
 (segment (start 160.337 123.698) (end 160.528 123.507) (width 0.25) (layer "F.Cu") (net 1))
 (segment (start 157.734 123.698) (end 160.337 123.698) (width 0.25) (layer "F.Cu") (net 1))
 (segment (start 157.415 114.173) (end 157.415 113.349) (width 0.25) (layer "F.Cu") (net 5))
 (segment (start 157.415 113.349) (end 157.5415 113.2225) (width 0.25) (layer "F.Cu") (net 5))
 (segment (start 157.5415 113.2225) (end 157.5415 112.014) (width 0.25) (layer "F.Cu") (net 5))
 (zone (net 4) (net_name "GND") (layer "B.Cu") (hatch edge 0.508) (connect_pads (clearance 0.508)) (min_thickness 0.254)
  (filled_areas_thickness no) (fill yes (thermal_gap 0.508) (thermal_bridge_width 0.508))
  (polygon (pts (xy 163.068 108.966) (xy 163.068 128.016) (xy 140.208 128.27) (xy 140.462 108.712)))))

